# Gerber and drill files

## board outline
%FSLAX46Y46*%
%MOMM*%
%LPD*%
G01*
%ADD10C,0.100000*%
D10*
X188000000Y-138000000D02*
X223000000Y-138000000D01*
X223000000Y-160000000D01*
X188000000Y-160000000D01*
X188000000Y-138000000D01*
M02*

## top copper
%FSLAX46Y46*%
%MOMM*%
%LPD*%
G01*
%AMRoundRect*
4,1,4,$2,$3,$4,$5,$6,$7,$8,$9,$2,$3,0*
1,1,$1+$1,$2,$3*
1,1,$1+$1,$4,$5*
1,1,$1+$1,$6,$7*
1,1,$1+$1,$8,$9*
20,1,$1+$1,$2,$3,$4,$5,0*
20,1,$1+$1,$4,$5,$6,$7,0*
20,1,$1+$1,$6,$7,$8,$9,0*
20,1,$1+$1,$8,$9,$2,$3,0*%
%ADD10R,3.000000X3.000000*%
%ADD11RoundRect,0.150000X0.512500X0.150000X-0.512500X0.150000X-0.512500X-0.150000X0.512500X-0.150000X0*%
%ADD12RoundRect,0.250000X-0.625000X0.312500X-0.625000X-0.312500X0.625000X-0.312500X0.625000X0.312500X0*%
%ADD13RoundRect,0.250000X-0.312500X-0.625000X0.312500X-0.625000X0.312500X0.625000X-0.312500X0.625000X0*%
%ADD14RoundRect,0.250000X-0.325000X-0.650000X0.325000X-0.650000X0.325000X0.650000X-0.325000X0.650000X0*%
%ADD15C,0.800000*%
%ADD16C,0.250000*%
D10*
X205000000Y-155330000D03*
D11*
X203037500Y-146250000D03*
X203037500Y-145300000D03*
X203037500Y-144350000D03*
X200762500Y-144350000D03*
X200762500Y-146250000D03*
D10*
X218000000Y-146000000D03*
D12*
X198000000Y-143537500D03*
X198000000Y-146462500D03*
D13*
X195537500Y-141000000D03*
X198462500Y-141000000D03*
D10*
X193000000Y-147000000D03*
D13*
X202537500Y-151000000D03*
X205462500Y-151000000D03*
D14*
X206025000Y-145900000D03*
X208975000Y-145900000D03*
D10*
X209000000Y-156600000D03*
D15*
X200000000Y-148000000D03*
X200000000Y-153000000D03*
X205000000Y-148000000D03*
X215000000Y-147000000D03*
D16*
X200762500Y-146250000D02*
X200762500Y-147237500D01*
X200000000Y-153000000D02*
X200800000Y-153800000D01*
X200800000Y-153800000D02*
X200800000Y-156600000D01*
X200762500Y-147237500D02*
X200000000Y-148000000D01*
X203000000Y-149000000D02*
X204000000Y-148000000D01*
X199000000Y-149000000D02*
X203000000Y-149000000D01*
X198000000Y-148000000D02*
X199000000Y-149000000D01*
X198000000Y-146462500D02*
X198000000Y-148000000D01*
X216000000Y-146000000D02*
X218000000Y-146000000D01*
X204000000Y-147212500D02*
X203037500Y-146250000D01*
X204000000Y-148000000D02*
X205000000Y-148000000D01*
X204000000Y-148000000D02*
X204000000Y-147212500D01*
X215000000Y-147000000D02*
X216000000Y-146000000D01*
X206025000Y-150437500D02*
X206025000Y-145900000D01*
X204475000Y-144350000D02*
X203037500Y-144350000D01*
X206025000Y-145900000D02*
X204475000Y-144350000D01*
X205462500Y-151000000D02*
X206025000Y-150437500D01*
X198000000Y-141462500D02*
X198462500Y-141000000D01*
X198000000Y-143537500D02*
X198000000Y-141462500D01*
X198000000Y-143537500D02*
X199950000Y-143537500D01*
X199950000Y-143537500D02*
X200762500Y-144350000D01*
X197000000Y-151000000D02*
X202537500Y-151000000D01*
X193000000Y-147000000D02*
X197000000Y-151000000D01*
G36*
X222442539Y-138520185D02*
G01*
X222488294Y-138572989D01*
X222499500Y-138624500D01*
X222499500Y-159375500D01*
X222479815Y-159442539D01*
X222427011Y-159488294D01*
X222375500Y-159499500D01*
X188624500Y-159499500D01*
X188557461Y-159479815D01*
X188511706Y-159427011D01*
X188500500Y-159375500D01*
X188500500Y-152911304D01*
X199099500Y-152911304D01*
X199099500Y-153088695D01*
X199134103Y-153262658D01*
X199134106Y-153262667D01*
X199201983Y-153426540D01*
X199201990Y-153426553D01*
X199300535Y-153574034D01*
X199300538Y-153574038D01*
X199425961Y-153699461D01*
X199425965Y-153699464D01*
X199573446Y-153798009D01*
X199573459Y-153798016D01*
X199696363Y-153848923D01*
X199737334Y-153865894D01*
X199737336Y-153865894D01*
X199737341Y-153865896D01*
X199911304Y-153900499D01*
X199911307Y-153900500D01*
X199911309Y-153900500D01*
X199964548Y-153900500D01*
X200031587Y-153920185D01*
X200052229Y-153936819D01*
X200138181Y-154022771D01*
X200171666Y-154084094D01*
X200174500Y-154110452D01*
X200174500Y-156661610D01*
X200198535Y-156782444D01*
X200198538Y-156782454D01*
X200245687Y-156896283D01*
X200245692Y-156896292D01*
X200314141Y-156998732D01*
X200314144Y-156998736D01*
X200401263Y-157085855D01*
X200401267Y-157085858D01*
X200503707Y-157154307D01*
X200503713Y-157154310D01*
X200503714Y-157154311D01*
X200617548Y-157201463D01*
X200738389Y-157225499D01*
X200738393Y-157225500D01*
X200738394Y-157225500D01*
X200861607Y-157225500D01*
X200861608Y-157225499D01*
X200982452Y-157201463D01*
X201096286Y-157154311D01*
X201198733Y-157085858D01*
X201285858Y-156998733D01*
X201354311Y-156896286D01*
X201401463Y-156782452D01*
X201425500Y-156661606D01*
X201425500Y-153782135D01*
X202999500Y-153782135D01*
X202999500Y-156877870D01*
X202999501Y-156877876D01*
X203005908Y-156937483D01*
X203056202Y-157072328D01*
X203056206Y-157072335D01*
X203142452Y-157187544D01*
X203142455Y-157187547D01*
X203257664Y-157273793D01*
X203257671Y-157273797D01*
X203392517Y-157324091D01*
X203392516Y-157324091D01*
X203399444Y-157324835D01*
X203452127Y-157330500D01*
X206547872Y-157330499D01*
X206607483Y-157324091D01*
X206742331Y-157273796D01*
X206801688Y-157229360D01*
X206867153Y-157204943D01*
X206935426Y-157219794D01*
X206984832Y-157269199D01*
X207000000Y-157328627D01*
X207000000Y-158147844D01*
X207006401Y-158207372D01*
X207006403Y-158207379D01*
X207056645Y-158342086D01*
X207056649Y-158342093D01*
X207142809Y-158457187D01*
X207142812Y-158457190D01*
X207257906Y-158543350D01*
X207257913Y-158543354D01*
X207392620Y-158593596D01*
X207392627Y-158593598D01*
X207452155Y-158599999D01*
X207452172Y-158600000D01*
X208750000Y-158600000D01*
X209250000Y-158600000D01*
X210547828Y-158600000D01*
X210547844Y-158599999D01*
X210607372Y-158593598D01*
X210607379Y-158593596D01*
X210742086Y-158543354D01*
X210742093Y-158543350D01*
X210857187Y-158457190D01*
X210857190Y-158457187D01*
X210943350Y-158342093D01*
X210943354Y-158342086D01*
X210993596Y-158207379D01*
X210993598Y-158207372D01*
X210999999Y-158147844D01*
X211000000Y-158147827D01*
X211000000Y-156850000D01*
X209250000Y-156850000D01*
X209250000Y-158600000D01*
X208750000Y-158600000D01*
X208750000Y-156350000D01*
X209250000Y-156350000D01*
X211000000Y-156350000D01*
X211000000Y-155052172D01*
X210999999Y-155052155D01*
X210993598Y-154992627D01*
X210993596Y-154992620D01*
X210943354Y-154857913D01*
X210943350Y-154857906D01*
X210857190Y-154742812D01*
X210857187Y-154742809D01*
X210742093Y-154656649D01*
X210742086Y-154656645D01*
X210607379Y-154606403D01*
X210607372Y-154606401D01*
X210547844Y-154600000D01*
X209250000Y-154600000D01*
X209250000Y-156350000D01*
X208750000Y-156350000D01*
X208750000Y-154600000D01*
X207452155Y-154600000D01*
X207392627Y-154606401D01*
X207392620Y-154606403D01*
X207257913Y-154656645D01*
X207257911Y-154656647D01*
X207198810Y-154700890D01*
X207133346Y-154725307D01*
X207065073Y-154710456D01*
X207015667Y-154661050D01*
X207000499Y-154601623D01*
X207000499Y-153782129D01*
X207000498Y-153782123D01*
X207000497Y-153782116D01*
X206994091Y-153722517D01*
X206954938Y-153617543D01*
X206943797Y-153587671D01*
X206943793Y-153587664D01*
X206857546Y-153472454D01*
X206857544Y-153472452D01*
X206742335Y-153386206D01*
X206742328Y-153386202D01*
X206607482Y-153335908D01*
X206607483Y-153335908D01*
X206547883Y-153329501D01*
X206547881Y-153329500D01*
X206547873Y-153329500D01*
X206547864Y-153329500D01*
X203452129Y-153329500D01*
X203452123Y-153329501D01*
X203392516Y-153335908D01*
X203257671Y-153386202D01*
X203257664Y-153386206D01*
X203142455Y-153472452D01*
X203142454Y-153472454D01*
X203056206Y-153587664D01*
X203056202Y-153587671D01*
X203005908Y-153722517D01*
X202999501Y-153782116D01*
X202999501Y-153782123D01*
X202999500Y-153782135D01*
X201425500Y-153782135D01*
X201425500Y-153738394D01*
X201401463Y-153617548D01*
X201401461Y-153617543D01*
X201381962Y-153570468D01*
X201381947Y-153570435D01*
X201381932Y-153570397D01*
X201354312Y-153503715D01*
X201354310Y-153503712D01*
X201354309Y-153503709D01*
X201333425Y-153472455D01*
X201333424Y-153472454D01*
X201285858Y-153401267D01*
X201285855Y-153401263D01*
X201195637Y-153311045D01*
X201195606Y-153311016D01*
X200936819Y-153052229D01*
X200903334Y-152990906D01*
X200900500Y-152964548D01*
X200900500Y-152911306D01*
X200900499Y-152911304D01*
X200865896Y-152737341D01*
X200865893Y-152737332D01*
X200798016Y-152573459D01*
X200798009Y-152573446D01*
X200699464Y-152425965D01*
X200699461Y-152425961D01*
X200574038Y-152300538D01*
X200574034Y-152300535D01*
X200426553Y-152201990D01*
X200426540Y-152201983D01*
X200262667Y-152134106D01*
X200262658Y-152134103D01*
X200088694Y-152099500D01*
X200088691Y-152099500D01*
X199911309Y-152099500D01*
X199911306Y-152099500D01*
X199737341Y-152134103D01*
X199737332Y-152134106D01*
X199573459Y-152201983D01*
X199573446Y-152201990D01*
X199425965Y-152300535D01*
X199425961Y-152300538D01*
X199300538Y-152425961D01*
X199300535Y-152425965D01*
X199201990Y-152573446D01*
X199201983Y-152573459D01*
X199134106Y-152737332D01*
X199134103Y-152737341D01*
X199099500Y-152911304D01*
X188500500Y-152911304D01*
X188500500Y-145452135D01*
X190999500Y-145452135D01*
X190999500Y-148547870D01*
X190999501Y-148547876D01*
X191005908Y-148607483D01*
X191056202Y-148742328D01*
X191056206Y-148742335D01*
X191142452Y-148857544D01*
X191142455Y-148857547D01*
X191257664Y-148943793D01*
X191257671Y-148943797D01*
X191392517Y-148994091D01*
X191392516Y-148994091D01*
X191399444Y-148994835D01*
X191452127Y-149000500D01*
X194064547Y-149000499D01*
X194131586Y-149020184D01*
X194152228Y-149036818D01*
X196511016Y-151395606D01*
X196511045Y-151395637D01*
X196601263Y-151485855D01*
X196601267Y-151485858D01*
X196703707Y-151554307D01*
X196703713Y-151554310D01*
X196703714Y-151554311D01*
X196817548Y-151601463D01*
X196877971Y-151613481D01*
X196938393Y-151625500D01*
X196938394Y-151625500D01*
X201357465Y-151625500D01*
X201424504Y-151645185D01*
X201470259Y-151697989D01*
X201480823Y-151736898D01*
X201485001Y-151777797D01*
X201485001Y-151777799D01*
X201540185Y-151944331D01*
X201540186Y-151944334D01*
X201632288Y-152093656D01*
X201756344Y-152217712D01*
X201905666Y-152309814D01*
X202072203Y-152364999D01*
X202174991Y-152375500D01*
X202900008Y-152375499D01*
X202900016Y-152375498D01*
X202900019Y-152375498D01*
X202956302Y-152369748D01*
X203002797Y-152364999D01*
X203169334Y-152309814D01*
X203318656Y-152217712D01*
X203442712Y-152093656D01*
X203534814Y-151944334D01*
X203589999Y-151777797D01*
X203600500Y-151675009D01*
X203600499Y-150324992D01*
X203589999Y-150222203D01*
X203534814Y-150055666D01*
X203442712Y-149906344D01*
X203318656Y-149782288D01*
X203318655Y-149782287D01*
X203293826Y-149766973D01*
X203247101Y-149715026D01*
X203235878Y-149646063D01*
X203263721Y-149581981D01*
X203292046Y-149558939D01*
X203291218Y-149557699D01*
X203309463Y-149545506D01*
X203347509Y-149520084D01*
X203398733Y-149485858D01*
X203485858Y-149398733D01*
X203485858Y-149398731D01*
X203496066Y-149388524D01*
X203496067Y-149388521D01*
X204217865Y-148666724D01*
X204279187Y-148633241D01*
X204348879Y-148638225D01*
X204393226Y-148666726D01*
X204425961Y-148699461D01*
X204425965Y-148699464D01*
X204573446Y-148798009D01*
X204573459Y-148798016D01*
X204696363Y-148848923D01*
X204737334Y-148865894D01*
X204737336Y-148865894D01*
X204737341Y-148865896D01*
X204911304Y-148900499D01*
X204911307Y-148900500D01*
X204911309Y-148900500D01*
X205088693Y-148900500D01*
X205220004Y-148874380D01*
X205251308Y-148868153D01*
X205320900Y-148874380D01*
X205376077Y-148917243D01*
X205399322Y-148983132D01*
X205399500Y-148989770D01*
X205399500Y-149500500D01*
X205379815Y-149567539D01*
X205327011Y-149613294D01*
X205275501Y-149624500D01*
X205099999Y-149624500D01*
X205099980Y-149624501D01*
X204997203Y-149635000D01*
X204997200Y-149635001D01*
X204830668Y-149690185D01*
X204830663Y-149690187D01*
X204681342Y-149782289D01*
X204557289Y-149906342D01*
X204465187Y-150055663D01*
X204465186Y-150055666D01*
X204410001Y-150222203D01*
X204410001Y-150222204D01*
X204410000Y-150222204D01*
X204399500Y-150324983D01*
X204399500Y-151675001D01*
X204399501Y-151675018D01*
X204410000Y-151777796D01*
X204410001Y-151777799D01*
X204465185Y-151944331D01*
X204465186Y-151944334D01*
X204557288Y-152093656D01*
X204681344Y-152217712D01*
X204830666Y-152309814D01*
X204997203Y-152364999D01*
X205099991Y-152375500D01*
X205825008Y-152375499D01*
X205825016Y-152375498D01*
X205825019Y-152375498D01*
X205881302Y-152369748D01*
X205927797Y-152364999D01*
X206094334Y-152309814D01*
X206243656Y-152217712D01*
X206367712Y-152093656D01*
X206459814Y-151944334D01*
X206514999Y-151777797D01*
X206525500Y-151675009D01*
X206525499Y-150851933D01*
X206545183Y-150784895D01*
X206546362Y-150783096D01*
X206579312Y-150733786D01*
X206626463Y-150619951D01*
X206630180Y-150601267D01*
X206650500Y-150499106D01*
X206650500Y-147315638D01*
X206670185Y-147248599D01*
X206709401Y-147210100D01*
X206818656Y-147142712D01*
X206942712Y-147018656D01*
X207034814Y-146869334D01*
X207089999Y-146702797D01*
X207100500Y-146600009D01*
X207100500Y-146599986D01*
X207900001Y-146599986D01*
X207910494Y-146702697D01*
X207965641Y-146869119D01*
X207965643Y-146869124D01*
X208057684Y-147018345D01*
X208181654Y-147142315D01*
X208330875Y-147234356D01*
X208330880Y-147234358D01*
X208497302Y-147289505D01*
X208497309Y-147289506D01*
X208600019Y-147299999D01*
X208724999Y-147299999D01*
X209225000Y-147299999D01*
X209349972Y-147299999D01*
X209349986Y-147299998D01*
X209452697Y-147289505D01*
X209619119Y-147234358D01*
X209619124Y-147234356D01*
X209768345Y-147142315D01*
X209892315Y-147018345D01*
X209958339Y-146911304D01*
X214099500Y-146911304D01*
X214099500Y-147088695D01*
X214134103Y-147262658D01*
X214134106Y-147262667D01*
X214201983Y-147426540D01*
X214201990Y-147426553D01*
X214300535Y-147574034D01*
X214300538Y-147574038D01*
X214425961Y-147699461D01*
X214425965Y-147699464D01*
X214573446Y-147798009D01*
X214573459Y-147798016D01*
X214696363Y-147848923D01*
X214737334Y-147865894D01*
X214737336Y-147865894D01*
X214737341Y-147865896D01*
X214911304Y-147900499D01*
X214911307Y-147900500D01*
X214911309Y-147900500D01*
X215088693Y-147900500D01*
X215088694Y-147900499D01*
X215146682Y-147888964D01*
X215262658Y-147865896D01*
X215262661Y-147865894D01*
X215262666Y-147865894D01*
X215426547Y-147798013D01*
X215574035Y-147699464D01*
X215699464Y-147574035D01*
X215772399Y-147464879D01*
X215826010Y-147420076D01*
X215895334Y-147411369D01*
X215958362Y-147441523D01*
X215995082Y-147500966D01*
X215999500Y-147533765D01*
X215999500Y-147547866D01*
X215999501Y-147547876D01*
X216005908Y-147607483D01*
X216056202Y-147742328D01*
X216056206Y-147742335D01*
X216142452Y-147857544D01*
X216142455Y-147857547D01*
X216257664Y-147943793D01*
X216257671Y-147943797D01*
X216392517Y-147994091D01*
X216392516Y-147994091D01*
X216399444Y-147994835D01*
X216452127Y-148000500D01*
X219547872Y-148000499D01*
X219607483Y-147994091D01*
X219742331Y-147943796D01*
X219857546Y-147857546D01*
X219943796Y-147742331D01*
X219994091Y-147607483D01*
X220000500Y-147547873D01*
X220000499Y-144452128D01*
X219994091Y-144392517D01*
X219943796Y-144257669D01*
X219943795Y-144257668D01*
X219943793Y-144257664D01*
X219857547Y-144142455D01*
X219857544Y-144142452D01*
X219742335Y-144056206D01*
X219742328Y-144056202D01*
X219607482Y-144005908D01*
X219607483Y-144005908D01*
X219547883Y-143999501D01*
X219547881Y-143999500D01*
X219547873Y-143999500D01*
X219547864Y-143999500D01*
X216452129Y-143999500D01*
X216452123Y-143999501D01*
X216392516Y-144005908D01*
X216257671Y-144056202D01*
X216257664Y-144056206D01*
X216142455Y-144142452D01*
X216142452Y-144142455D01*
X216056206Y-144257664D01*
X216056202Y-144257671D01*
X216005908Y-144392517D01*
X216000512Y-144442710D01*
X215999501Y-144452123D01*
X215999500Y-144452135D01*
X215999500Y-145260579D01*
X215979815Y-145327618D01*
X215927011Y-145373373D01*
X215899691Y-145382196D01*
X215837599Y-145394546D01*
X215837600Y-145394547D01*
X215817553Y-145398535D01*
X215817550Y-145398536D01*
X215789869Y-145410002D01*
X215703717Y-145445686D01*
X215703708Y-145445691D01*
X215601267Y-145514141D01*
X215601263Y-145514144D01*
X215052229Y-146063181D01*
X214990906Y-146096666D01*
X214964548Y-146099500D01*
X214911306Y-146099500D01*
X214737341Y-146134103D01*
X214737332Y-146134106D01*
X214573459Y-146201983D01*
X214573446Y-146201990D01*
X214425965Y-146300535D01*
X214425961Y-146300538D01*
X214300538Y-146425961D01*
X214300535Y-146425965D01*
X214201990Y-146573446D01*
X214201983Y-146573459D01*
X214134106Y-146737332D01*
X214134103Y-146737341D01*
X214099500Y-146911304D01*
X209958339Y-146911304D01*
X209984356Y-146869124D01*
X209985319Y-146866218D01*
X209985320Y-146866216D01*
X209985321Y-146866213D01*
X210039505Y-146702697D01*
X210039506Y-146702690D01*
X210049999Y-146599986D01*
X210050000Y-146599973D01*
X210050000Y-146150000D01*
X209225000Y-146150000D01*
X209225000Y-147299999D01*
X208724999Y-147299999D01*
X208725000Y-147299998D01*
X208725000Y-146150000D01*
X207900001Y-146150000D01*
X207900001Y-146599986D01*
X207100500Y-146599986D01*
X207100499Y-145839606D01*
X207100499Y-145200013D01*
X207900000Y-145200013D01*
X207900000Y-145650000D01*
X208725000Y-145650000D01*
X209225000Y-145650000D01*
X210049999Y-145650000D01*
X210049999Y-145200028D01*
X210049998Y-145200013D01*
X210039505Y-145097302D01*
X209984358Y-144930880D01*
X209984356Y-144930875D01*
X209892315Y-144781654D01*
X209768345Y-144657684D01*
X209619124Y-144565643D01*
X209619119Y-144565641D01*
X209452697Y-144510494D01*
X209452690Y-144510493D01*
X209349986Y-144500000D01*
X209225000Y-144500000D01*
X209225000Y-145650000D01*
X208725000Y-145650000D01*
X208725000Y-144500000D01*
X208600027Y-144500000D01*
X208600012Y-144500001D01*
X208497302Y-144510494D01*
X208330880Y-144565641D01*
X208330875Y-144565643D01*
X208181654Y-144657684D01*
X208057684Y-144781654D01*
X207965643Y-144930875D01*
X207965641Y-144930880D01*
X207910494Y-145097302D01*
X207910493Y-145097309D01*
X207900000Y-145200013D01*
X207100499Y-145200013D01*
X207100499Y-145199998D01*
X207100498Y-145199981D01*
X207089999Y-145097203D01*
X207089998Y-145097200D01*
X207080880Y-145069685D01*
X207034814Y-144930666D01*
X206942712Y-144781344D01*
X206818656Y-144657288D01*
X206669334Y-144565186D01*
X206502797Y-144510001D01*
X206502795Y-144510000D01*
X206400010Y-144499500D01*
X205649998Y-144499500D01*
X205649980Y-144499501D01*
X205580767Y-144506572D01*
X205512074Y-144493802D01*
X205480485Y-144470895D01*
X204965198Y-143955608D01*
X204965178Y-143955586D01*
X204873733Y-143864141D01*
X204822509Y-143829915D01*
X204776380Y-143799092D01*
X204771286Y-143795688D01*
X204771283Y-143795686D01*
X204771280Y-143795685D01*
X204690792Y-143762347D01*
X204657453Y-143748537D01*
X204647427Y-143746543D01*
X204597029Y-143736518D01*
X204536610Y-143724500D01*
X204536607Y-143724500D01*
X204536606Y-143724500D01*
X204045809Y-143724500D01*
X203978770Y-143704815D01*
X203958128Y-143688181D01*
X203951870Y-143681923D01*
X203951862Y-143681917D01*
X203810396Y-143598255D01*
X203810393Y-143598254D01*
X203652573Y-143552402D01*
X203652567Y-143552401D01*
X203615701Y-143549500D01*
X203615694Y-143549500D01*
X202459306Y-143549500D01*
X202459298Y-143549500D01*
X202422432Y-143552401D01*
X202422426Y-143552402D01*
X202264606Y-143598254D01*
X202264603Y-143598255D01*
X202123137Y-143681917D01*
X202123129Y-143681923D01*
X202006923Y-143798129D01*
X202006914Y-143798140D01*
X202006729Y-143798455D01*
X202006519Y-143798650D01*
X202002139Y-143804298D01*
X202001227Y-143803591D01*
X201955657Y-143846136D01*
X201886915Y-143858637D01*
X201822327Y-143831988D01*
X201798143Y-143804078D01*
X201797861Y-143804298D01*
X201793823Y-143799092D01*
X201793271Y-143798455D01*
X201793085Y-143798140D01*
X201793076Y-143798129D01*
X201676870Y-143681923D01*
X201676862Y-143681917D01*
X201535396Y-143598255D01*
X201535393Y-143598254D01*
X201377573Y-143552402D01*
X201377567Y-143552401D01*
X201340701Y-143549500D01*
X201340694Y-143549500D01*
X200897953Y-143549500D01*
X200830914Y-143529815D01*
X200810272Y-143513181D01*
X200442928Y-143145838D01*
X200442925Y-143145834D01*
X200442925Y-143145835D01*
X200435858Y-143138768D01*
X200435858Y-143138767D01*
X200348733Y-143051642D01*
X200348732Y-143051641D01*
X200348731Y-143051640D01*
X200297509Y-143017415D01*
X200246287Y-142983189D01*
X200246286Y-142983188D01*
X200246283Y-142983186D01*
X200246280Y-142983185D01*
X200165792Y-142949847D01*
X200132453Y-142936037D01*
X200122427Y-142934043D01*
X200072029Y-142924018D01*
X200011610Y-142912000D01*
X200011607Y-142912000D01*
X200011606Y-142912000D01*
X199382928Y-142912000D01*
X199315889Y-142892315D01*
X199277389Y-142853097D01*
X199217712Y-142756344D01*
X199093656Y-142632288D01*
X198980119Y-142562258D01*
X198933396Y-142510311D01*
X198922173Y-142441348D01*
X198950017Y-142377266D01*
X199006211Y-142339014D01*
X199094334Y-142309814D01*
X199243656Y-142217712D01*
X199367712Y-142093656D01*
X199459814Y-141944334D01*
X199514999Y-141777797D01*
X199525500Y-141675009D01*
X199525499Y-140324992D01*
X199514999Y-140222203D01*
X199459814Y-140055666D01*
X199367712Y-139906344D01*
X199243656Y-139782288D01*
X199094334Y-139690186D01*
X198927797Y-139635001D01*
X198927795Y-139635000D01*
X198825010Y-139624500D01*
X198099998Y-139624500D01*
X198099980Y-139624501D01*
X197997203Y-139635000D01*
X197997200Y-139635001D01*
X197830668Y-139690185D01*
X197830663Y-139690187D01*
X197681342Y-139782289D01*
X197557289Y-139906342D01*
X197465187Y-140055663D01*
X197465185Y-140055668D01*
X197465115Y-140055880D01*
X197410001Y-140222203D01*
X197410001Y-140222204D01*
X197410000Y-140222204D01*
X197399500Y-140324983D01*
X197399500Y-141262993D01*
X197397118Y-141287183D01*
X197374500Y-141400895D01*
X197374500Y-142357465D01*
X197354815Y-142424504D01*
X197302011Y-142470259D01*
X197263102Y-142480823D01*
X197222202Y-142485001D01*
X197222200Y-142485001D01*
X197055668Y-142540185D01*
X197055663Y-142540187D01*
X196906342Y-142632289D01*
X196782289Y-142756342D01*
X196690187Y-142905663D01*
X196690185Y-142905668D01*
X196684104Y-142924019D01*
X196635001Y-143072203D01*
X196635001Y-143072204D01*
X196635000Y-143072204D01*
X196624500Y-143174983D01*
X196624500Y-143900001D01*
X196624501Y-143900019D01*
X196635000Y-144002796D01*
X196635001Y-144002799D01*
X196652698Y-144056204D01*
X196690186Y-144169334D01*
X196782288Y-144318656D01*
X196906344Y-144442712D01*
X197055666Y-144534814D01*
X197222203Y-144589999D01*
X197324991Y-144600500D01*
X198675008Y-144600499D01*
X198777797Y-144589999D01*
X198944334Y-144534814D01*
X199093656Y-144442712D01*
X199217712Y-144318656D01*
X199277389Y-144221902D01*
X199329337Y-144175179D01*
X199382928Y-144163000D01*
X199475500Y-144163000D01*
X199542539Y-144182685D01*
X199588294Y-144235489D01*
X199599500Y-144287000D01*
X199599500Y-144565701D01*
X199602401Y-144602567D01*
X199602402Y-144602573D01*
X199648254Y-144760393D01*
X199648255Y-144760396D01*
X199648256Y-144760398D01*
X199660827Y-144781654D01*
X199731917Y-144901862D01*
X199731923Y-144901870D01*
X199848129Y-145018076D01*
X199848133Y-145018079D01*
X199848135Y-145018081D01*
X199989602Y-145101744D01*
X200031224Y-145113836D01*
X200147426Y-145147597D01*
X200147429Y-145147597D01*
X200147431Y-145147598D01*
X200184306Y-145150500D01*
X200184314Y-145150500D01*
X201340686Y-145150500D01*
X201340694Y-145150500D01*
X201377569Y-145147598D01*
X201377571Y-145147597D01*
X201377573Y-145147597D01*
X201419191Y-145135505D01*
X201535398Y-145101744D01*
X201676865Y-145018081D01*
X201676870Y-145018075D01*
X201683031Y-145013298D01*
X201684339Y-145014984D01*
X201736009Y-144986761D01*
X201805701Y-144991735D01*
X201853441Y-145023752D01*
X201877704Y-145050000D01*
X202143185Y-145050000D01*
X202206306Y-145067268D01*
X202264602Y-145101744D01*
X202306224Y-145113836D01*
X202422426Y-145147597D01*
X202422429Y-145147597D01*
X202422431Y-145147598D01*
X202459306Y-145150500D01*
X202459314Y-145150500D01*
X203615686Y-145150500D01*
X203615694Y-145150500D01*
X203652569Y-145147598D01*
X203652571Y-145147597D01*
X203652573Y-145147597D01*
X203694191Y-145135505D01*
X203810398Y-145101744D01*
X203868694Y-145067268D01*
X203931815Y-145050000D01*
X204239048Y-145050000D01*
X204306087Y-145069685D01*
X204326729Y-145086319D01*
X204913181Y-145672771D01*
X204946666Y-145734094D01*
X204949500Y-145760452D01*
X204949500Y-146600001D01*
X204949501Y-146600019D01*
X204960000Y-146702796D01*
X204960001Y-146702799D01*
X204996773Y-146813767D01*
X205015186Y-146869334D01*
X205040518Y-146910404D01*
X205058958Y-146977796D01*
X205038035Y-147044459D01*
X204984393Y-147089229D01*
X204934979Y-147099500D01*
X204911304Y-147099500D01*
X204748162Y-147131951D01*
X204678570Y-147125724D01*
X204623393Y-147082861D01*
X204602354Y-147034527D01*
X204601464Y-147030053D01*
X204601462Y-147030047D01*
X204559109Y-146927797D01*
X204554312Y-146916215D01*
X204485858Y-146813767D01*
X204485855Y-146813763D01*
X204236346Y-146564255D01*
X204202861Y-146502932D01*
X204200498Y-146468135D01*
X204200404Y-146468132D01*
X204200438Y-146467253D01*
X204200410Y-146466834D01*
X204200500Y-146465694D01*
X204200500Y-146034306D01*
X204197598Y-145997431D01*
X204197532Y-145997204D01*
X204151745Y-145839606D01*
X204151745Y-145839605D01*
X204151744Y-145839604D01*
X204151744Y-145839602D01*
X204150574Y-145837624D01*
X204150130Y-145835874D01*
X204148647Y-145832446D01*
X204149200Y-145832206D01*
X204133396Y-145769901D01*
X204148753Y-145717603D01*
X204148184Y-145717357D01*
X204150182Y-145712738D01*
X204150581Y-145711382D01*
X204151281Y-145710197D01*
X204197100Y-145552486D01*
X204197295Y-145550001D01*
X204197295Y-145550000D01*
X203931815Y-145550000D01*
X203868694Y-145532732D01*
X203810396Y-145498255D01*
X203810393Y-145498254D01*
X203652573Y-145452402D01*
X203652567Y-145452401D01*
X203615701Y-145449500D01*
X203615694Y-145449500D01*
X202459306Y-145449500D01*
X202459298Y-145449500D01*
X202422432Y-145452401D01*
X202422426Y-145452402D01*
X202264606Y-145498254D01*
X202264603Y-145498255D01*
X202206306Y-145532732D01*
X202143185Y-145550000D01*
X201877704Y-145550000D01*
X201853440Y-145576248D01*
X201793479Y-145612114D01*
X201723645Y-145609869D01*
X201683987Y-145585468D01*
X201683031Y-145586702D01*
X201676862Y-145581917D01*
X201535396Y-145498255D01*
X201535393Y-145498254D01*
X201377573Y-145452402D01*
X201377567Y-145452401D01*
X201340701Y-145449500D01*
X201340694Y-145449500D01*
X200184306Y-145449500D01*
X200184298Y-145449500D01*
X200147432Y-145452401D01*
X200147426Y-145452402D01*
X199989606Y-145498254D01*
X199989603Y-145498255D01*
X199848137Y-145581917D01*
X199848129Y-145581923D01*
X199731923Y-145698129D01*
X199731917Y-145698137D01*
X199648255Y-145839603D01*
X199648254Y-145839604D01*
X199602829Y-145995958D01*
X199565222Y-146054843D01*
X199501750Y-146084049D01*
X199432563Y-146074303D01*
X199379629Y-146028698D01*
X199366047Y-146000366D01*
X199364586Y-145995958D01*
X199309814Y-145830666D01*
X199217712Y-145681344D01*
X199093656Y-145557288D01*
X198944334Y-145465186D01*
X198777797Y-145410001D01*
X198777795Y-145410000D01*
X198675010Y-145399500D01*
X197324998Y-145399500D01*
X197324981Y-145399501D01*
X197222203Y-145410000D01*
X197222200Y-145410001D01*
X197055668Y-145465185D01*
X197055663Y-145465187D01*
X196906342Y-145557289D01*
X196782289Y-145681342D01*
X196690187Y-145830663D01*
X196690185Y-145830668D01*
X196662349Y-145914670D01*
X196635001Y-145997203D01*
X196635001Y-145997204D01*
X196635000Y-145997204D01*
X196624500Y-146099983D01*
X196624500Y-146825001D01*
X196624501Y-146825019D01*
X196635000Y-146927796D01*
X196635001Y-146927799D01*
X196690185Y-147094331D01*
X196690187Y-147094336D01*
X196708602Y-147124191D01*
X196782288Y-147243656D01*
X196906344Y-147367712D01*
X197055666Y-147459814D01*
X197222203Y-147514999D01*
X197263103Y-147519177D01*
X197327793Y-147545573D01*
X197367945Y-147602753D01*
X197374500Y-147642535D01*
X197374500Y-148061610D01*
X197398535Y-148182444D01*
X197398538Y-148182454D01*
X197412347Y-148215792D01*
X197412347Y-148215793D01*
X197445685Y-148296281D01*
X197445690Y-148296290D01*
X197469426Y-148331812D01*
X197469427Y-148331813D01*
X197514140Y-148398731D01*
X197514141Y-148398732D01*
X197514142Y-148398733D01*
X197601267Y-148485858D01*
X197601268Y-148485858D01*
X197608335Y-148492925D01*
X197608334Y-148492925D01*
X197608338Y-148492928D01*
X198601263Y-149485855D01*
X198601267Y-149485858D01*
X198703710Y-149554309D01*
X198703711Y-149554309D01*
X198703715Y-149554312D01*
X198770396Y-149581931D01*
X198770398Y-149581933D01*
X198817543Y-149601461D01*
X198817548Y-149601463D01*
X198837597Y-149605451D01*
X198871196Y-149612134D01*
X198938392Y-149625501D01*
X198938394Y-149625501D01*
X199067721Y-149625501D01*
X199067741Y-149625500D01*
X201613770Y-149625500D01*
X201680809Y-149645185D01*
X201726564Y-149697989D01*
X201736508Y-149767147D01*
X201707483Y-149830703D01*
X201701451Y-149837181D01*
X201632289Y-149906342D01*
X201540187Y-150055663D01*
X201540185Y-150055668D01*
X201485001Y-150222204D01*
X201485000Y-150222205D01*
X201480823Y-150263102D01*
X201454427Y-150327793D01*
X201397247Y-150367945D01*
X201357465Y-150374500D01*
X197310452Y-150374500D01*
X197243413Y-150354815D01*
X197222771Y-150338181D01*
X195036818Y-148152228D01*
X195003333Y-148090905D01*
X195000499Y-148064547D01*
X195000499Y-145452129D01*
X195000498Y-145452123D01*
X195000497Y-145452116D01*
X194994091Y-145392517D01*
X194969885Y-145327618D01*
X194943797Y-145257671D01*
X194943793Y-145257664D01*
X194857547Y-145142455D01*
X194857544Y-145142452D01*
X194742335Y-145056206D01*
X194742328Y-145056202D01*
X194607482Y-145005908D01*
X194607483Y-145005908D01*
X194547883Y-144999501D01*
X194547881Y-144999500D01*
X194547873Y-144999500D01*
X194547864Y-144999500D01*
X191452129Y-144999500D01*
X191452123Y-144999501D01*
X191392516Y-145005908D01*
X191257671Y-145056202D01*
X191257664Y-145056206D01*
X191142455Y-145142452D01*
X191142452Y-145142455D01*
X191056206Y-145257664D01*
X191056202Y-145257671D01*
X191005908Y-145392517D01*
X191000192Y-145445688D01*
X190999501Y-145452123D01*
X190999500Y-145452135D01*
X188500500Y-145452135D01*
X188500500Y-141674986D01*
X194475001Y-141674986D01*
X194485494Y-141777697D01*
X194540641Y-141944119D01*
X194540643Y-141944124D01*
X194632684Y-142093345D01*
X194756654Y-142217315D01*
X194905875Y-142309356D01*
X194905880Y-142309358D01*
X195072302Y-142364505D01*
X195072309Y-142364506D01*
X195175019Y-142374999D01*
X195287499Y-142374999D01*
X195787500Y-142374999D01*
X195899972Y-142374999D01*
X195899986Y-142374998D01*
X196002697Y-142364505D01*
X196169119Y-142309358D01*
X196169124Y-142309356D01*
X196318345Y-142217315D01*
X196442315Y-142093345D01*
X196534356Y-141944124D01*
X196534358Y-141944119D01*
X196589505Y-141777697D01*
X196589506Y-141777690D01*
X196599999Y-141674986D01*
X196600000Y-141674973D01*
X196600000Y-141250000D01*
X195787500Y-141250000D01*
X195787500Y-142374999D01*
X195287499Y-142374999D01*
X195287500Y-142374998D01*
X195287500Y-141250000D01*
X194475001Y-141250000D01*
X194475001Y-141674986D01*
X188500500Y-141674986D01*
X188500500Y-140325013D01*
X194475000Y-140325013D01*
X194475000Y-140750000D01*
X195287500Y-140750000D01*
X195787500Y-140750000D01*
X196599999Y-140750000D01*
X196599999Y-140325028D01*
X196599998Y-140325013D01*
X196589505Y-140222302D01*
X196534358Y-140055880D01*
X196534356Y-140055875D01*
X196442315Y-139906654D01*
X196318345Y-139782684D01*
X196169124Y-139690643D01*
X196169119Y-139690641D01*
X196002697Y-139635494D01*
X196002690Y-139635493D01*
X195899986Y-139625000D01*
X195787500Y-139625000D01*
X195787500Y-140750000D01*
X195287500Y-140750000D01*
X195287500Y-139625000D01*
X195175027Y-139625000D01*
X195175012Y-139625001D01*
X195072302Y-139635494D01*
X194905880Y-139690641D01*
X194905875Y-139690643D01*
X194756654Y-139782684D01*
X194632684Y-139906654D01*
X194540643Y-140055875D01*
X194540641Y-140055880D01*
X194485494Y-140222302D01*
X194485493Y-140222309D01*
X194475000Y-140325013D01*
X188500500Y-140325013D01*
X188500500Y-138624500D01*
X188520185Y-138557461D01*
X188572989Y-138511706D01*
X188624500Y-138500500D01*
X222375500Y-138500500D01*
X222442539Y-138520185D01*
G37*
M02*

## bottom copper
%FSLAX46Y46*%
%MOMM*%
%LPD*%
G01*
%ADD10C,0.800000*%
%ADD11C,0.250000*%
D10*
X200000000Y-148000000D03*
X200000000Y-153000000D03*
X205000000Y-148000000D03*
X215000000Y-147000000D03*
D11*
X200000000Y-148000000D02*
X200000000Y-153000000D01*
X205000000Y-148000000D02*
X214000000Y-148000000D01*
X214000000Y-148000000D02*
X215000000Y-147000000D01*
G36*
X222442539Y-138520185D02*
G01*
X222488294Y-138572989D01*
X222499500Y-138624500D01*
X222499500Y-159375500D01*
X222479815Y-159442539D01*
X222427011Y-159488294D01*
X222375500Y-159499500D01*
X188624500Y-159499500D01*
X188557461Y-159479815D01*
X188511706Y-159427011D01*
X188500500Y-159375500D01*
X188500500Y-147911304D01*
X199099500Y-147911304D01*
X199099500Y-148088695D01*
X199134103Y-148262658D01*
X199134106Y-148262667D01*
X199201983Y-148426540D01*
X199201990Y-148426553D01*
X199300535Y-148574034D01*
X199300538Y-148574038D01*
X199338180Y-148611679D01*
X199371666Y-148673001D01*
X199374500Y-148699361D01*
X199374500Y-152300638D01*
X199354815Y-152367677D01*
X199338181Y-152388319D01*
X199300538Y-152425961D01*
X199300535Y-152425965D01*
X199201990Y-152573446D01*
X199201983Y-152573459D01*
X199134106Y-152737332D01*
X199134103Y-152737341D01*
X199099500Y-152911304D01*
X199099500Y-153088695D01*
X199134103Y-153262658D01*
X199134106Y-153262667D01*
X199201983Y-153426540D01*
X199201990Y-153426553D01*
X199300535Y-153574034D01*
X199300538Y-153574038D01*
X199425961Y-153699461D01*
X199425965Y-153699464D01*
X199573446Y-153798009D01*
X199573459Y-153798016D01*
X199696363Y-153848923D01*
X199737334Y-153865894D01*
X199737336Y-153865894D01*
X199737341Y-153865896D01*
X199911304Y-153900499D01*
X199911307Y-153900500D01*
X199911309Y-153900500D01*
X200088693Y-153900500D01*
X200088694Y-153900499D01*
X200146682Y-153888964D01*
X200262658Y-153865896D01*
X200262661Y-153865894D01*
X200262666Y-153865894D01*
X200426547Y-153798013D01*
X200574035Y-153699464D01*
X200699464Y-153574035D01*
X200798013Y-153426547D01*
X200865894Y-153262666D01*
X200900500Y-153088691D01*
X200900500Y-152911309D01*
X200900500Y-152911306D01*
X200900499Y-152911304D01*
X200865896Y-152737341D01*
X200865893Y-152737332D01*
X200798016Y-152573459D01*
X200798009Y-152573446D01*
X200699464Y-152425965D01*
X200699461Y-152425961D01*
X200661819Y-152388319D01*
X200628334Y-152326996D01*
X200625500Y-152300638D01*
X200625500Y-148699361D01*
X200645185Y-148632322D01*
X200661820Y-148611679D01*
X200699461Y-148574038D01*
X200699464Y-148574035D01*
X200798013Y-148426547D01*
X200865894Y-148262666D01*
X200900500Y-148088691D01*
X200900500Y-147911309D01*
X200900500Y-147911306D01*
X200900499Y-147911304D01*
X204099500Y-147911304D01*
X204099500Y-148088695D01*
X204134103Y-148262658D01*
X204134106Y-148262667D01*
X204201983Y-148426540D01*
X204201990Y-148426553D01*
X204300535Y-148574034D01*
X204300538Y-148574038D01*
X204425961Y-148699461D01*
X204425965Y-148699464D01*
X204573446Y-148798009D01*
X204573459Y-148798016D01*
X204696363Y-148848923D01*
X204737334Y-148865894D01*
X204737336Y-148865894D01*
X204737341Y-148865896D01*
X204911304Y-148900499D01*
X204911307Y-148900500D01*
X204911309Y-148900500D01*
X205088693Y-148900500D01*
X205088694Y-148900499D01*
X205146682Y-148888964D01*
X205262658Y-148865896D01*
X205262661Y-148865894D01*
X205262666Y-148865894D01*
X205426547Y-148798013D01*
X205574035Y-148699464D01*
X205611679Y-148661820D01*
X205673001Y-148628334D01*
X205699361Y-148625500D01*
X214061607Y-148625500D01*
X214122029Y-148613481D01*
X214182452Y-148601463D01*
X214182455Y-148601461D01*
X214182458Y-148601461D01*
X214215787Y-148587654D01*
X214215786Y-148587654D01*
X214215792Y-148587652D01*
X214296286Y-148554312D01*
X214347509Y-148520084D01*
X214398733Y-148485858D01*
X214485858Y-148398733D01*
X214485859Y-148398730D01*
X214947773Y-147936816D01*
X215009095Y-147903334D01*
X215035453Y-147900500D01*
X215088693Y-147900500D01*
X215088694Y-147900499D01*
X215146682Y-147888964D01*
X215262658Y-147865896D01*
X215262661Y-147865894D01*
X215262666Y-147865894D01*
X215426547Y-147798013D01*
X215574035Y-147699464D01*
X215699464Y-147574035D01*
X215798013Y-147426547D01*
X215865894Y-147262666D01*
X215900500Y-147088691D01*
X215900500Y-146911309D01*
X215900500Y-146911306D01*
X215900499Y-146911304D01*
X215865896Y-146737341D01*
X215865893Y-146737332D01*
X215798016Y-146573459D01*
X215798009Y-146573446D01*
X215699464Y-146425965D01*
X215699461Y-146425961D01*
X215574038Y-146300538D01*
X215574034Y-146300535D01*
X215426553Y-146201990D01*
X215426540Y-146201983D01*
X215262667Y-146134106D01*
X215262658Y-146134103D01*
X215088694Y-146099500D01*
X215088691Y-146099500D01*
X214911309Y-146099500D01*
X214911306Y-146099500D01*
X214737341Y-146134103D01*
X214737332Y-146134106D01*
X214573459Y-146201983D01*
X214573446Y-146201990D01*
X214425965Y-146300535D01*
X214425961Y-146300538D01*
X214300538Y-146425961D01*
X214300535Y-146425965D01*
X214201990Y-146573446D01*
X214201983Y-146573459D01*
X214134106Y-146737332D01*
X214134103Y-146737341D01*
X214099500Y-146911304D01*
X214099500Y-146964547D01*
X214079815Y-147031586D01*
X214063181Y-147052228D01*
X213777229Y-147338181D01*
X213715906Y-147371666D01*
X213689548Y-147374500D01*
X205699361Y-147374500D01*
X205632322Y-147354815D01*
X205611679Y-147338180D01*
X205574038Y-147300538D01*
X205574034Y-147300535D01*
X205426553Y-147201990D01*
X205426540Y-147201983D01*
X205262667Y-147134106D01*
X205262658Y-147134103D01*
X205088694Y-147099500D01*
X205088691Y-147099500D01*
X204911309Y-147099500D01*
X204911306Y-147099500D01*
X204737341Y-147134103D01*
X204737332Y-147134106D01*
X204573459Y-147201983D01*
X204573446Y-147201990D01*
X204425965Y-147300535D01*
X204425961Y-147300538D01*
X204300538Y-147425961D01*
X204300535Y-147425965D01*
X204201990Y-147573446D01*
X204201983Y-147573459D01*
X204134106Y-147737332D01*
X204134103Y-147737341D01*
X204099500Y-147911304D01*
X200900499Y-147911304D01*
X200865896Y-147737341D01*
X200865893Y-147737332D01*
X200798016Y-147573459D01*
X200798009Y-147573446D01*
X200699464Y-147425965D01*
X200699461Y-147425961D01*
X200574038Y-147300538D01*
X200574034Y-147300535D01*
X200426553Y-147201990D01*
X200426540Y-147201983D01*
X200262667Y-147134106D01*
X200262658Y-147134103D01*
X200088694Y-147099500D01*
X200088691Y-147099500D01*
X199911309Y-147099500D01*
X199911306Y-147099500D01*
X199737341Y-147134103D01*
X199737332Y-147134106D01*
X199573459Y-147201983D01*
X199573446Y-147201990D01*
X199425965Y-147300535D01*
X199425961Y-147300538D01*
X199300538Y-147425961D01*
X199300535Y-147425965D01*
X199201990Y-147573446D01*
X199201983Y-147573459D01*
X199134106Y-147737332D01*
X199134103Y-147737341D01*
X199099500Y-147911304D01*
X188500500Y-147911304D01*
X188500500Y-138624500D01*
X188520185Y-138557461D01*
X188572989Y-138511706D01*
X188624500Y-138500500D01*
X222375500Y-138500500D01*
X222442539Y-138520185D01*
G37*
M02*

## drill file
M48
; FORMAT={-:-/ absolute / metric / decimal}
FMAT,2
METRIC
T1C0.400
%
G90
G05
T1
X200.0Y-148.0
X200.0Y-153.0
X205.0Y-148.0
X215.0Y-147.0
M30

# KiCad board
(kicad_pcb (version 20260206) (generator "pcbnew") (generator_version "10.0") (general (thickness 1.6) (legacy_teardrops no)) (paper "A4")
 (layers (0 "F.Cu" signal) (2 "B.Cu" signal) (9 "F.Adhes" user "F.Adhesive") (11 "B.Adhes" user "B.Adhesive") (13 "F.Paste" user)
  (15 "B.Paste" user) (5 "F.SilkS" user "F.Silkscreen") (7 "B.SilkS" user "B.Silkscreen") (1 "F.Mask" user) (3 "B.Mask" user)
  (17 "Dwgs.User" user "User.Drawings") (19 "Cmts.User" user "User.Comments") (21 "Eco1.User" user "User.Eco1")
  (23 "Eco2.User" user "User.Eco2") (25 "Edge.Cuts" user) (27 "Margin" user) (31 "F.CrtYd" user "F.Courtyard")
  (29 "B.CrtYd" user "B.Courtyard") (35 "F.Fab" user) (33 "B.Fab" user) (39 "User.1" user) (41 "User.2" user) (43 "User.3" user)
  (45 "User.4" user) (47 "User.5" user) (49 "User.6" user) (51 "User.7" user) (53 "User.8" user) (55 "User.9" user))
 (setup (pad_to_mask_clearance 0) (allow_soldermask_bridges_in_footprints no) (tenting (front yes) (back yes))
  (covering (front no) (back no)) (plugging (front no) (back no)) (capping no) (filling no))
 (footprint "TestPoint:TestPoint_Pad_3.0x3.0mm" (layer "F.Cu") (at 205 155.33)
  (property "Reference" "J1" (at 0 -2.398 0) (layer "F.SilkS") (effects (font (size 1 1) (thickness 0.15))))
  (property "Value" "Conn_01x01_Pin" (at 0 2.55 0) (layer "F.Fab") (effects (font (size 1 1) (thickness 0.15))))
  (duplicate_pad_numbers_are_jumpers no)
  (pad "1" smd rect (at 0 0) (size 3 3) (layers "F.Cu" "F.Mask") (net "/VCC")))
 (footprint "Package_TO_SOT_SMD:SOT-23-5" (layer "F.Cu") (at 201.9 145.3 180)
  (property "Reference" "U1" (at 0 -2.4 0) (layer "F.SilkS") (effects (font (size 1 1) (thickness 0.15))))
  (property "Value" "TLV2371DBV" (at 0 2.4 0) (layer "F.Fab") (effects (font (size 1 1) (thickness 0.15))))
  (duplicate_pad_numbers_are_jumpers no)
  (pad "1" smd roundrect (at -1.1375 -0.95 180) (size 1.325 0.6) (layers "F.Cu" "F.Mask" "F.Paste") (roundrect_rratio 0.25) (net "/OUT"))
  (pad "2" smd roundrect (at -1.1375 0 180) (size 1.325 0.6) (layers "F.Cu" "F.Mask" "F.Paste") (roundrect_rratio 0.25) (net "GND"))
  (pad "3" smd roundrect (at -1.1375 0.95 180) (size 1.325 0.6) (layers "F.Cu" "F.Mask" "F.Paste") (roundrect_rratio 0.25)
   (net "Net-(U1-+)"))
  (pad "4" smd roundrect (at 1.1375 0.95 180) (size 1.325 0.6) (layers "F.Cu" "F.Mask" "F.Paste") (roundrect_rratio 0.25) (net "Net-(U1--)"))
  (pad "5" smd roundrect (at 1.1375 -0.95 180) (size 1.325 0.6) (layers "F.Cu" "F.Mask" "F.Paste") (roundrect_rratio 0.25) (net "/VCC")))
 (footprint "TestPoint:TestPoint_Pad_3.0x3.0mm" (layer "F.Cu") (at 218 146)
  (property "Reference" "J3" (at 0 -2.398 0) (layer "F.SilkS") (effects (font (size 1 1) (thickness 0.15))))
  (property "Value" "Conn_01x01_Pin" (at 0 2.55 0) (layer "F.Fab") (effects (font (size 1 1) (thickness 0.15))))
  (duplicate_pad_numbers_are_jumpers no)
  (pad "1" smd rect (at 0 0) (size 3 3) (layers "F.Cu" "F.Mask") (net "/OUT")))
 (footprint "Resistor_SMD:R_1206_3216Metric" (layer "F.Cu") (at 198 145 -90)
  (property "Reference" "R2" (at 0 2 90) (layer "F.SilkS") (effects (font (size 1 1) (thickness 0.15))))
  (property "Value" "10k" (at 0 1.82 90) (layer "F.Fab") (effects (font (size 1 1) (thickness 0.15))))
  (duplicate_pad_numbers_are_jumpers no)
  (pad "1" smd roundrect (at -1.4625 0 270) (size 1.125 1.75) (layers "F.Cu" "F.Mask" "F.Paste") (roundrect_rratio 0.222222)
   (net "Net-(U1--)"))
  (pad "2" smd roundrect (at 1.4625 0 270) (size 1.125 1.75) (layers "F.Cu" "F.Mask" "F.Paste") (roundrect_rratio 0.222222) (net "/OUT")))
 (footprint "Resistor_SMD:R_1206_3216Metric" (layer "F.Cu") (at 197 141)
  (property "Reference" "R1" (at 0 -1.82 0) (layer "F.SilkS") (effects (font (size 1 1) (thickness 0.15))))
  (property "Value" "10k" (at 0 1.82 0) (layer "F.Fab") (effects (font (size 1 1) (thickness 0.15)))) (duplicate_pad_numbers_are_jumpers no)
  (pad "1" smd roundrect (at -1.4625 0) (size 1.125 1.75) (layers "F.Cu" "F.Mask" "F.Paste") (roundrect_rratio 0.222222) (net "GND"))
  (pad "2" smd roundrect (at 1.4625 0) (size 1.125 1.75) (layers "F.Cu" "F.Mask" "F.Paste") (roundrect_rratio 0.222222) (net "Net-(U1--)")))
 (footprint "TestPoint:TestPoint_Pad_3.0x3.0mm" (layer "F.Cu") (at 193 147)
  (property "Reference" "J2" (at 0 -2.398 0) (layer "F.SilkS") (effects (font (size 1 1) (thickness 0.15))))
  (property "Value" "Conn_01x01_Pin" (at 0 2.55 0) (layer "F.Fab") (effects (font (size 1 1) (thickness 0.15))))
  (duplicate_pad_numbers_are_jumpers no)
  (pad "1" smd rect (at 0 0) (size 3 3) (layers "F.Cu" "F.Mask") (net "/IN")))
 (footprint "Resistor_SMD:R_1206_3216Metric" (layer "F.Cu") (at 204 151)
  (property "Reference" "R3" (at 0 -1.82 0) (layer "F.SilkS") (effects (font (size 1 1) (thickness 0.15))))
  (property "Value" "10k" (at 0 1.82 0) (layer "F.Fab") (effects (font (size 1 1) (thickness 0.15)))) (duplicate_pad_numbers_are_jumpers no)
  (pad "1" smd roundrect (at -1.4625 0) (size 1.125 1.75) (layers "F.Cu" "F.Mask" "F.Paste") (roundrect_rratio 0.222222) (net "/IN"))
  (pad "2" smd roundrect (at 1.4625 0) (size 1.125 1.75) (layers "F.Cu" "F.Mask" "F.Paste") (roundrect_rratio 0.222222) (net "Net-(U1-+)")))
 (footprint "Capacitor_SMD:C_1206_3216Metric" (layer "F.Cu") (at 207.5 145.9)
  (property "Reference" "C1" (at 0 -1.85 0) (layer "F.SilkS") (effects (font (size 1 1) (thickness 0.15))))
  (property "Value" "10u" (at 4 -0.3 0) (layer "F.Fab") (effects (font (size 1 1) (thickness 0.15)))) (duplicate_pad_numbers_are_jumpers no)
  (pad "1" smd roundrect (at -1.475 0) (size 1.15 1.8) (layers "F.Cu" "F.Mask" "F.Paste") (roundrect_rratio 0.217391) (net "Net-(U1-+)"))
  (pad "2" smd roundrect (at 1.475 0) (size 1.15 1.8) (layers "F.Cu" "F.Mask" "F.Paste") (roundrect_rratio 0.217391) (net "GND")))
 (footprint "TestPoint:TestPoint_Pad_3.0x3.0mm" (layer "F.Cu") (at 209 156.6)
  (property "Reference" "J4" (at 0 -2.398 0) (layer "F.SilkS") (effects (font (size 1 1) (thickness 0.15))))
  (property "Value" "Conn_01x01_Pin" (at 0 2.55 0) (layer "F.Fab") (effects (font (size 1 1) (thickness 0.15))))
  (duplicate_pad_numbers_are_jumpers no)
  (pad "1" smd rect (at 0 0) (size 3 3) (layers "F.Cu" "F.Mask") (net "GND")))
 (gr_rect (start 188 138) (end 223 160) (stroke (width 0.1) (type default)) (fill no) (layer "Edge.Cuts"))
 (segment (start 200.7625 146.25) (end 200.7625 147.2375) (width 0.25) (layer "F.Cu") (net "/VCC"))
 (segment (start 200 153) (end 200.8 153.8) (width 0.25) (layer "F.Cu") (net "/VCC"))
 (segment (start 200.8 153.8) (end 200.8 156.6) (width 0.25) (layer "F.Cu") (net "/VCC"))
 (segment (start 200.7625 147.2375) (end 200 148) (width 0.25) (layer "F.Cu") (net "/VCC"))
 (via (at 200 148) (size 0.8) (drill 0.4) (layers "F.Cu" "B.Cu") (capping no) (covering (front no) (back no))
  (plugging (front no) (back no)) (filling no) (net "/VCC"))
 (via (at 200 153) (size 0.8) (drill 0.4) (layers "F.Cu" "B.Cu") (capping no) (covering (front no) (back no))
  (plugging (front no) (back no)) (filling no) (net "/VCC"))
 (segment (start 200 148) (end 200 153) (width 0.25) (layer "B.Cu") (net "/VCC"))
 (segment (start 203 149) (end 204 148) (width 0.25) (layer "F.Cu") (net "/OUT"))
 (segment (start 199 149) (end 203 149) (width 0.25) (layer "F.Cu") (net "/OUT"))
 (segment (start 198 148) (end 199 149) (width 0.25) (layer "F.Cu") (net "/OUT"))
 (segment (start 198 146.4625) (end 198 148) (width 0.25) (layer "F.Cu") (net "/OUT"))
 (segment (start 216 146) (end 218 146) (width 0.25) (layer "F.Cu") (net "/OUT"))
 (segment (start 204 147.2125) (end 203.0375 146.25) (width 0.25) (layer "F.Cu") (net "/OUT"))
 (segment (start 204 148) (end 205 148) (width 0.25) (layer "F.Cu") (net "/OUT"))
 (segment (start 204 148) (end 204 147.2125) (width 0.25) (layer "F.Cu") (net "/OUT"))
 (segment (start 215 147) (end 216 146) (width 0.25) (layer "F.Cu") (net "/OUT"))
 (via (at 205 148) (size 0.8) (drill 0.4) (layers "F.Cu" "B.Cu") (capping no) (covering (front no) (back no))
  (plugging (front no) (back no)) (filling no) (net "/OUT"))
 (via (at 215 147) (size 0.8) (drill 0.4) (layers "F.Cu" "B.Cu") (capping no) (covering (front no) (back no))
  (plugging (front no) (back no)) (filling no) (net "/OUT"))
 (segment (start 205 148) (end 214 148) (width 0.25) (layer "B.Cu") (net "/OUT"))
 (segment (start 214 148) (end 215 147) (width 0.25) (layer "B.Cu") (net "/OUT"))
 (segment (start 206.025 150.4375) (end 206.025 145.9) (width 0.25) (layer "F.Cu") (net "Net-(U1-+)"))
 (segment (start 204.475 144.35) (end 203.0375 144.35) (width 0.25) (layer "F.Cu") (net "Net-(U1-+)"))
 (segment (start 206.025 145.9) (end 204.475 144.35) (width 0.25) (layer "F.Cu") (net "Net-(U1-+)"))
 (segment (start 205.4625 151) (end 206.025 150.4375) (width 0.25) (layer "F.Cu") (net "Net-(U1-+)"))
 (segment (start 198 141.4625) (end 198.4625 141) (width 0.25) (layer "F.Cu") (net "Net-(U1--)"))
 (segment (start 198 143.5375) (end 198 141.4625) (width 0.25) (layer "F.Cu") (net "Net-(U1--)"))
 (segment (start 198 143.5375) (end 199.95 143.5375) (width 0.25) (layer "F.Cu") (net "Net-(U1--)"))
 (segment (start 199.95 143.5375) (end 200.7625 144.35) (width 0.25) (layer "F.Cu") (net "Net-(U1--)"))
 (segment (start 197 151) (end 202.5375 151) (width 0.25) (layer "F.Cu") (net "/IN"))
 (segment (start 193 147) (end 197 151) (width 0.25) (layer "F.Cu") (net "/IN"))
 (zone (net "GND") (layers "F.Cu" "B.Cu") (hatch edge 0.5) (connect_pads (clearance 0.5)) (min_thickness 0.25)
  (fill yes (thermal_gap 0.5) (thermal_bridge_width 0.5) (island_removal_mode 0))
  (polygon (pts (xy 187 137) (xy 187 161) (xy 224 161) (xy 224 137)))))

